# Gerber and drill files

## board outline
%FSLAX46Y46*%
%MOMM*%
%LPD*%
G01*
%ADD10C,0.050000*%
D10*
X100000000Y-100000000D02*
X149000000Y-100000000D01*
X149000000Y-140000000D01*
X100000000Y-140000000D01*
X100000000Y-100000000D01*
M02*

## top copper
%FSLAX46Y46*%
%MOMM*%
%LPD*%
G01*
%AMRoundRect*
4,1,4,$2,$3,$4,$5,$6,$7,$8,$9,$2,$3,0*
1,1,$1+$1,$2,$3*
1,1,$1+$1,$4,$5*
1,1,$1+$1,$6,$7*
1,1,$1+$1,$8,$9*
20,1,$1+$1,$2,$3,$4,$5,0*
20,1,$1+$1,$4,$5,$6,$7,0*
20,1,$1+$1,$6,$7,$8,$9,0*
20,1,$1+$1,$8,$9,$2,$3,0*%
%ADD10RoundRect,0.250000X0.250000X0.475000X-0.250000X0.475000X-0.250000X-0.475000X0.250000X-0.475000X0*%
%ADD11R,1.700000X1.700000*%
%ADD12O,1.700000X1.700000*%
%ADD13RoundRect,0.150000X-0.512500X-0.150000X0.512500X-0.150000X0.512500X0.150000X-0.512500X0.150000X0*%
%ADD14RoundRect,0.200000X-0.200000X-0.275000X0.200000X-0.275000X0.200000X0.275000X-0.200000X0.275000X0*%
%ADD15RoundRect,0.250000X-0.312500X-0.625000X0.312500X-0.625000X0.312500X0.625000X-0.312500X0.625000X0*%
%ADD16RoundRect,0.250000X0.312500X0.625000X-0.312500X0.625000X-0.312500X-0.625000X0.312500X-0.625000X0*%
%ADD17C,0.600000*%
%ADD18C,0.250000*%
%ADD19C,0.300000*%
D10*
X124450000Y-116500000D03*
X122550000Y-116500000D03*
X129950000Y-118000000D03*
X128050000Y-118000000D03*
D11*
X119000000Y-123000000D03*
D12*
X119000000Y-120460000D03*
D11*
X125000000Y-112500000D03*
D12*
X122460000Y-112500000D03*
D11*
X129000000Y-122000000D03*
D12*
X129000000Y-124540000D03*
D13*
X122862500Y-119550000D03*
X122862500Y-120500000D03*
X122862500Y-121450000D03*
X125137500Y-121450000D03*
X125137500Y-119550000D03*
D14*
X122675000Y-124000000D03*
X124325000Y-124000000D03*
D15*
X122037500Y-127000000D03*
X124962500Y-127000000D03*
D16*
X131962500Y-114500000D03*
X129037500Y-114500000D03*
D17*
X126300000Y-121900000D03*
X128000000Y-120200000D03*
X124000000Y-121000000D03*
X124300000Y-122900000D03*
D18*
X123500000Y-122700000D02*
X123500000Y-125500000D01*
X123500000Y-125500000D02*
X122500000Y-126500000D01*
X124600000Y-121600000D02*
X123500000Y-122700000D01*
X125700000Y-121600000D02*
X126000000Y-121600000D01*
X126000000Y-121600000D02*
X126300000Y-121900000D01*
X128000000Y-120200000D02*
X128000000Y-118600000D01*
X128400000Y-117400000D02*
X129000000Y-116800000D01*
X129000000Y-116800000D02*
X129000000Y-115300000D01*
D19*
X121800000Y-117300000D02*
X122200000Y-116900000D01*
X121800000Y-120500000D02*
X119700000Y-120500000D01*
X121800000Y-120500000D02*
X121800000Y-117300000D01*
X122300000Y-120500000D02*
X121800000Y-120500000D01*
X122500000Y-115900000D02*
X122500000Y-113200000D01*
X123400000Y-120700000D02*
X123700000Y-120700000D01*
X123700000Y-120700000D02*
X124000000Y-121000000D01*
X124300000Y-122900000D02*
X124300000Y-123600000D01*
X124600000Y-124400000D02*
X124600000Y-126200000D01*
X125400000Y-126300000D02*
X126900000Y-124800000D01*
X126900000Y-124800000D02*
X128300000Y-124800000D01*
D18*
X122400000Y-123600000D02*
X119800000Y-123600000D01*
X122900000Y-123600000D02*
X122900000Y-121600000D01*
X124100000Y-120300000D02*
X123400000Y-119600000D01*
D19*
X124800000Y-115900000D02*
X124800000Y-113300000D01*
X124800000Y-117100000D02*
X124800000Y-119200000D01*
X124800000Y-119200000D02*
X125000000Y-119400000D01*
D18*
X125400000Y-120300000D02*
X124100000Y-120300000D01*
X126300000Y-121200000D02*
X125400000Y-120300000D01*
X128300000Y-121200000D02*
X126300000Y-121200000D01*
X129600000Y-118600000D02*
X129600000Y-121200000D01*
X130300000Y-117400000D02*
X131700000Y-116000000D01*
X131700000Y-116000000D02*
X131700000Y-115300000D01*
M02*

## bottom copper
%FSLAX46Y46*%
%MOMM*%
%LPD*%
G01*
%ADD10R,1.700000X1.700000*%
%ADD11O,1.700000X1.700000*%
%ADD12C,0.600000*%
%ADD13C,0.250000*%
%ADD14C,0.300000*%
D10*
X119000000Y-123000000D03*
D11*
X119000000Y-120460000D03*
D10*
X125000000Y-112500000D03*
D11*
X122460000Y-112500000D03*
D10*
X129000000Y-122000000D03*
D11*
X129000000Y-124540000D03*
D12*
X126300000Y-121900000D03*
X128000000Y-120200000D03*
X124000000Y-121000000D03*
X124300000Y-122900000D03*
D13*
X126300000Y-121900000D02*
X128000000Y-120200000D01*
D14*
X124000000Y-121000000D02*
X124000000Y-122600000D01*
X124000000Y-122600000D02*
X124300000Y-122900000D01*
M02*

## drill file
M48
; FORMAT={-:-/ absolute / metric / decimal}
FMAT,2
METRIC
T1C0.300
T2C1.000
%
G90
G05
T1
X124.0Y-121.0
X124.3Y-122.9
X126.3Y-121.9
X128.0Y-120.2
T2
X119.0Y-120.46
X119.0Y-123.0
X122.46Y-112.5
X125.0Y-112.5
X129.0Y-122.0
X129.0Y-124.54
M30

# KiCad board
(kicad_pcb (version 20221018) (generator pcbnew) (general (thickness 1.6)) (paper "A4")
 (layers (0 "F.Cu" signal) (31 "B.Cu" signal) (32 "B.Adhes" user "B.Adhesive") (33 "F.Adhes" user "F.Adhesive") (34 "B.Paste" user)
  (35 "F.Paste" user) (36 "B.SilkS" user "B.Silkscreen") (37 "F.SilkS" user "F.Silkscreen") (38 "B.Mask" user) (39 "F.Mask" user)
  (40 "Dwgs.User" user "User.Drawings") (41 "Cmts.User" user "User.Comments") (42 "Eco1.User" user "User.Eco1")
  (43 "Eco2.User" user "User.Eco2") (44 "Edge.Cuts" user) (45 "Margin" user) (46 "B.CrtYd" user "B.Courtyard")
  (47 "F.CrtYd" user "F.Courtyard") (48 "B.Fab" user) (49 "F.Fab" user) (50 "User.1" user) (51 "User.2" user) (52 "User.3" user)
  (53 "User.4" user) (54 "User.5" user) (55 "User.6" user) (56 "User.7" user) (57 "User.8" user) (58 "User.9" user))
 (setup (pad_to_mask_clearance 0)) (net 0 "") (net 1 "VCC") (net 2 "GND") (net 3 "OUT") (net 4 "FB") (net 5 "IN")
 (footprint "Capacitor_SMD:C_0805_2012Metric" (layer "F.Cu") (at 123.5 116.5 180)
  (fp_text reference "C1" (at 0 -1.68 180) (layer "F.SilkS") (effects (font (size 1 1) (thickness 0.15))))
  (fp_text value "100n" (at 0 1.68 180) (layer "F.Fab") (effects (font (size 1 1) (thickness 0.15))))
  (pad "1" smd roundrect (at -0.95 0 180) (size 1 1.45) (layers "F.Cu" "F.Paste" "F.Mask") (roundrect_rratio 0.25) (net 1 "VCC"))
  (pad "2" smd roundrect (at 0.95 0 180) (size 1 1.45) (layers "F.Cu" "F.Paste" "F.Mask") (roundrect_rratio 0.25) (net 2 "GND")))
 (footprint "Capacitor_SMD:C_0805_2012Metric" (layer "F.Cu") (at 129 118 180)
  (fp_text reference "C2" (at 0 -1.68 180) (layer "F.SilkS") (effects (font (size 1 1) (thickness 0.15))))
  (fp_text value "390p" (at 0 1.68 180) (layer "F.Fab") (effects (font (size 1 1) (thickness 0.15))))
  (pad "1" smd roundrect (at -0.95 0 180) (size 1 1.45) (layers "F.Cu" "F.Paste" "F.Mask") (roundrect_rratio 0.25) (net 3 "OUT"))
  (pad "2" smd roundrect (at 0.95 0 180) (size 1 1.45) (layers "F.Cu" "F.Paste" "F.Mask") (roundrect_rratio 0.25) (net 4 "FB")))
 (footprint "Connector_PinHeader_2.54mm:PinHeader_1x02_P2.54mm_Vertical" (layer "F.Cu") (at 119 123 180)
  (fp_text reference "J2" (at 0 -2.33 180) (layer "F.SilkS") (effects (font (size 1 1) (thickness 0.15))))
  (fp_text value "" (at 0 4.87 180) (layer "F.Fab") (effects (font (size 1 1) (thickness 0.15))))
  (pad "1" thru_hole rect (at 0 0 180) (size 1.7 1.7) (drill 1) (layers "*.Cu" "*.Mask") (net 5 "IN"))
  (pad "2" thru_hole oval (at 0 2.54 180) (size 1.7 1.7) (drill 1) (layers "*.Cu" "*.Mask") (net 2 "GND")))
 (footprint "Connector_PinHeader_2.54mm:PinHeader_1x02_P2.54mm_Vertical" (layer "F.Cu") (at 125 112.5 -90)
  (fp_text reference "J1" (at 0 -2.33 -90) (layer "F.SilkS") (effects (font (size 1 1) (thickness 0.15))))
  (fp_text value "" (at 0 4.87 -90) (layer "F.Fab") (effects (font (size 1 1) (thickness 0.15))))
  (pad "1" thru_hole rect (at 0 0 270) (size 1.7 1.7) (drill 1) (layers "*.Cu" "*.Mask") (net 1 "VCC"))
  (pad "2" thru_hole oval (at 0 2.54 270) (size 1.7 1.7) (drill 1) (layers "*.Cu" "*.Mask") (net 2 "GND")))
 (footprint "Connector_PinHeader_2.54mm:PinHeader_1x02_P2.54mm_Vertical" (layer "F.Cu") (at 129 122)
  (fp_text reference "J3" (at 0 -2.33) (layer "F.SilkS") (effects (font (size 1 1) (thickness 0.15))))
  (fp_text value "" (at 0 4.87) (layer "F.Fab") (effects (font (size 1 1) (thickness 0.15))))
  (pad "1" thru_hole rect (at 0 0) (size 1.7 1.7) (drill 1) (layers "*.Cu" "*.Mask") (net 3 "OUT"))
  (pad "2" thru_hole oval (at 0 2.54) (size 1.7 1.7) (drill 1) (layers "*.Cu" "*.Mask") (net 2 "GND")))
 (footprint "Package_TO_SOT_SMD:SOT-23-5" (layer "F.Cu") (at 124 120.5)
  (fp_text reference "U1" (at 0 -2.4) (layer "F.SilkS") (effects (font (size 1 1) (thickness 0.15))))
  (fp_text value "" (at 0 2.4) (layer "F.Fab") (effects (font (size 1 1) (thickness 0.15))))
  (pad "1" smd roundrect (at -1.1375 -0.95) (size 1.325 0.6) (layers "F.Cu" "F.Paste" "F.Mask") (roundrect_rratio 0.25) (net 3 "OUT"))
  (pad "2" smd roundrect (at -1.1375 0) (size 1.325 0.6) (layers "F.Cu" "F.Paste" "F.Mask") (roundrect_rratio 0.25) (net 2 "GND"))
  (pad "3" smd roundrect (at -1.1375 0.95) (size 1.325 0.6) (layers "F.Cu" "F.Paste" "F.Mask") (roundrect_rratio 0.25) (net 5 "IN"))
  (pad "4" smd roundrect (at 1.1375 0.95) (size 1.325 0.6) (layers "F.Cu" "F.Paste" "F.Mask") (roundrect_rratio 0.25) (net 4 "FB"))
  (pad "5" smd roundrect (at 1.1375 -0.95) (size 1.325 0.6) (layers "F.Cu" "F.Paste" "F.Mask") (roundrect_rratio 0.25) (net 1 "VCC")))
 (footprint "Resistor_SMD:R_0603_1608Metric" (layer "F.Cu") (at 123.5 124)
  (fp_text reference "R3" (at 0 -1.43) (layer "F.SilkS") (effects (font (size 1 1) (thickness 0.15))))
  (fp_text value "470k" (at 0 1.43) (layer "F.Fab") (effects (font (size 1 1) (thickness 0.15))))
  (pad "1" smd roundrect (at -0.825 0) (size 0.8 0.95) (layers "F.Cu" "F.Paste" "F.Mask") (roundrect_rratio 0.25) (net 5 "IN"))
  (pad "2" smd roundrect (at 0.825 0) (size 0.8 0.95) (layers "F.Cu" "F.Paste" "F.Mask") (roundrect_rratio 0.25) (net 2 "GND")))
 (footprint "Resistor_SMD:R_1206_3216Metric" (layer "F.Cu") (at 123.5 127)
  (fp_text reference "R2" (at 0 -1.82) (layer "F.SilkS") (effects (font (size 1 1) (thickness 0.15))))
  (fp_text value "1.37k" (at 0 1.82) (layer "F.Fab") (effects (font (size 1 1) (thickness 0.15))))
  (pad "1" smd roundrect (at -1.4625 0) (size 1.125 1.75) (layers "F.Cu" "F.Paste" "F.Mask") (roundrect_rratio 0.222222) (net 4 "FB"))
  (pad "2" smd roundrect (at 1.4625 0) (size 1.125 1.75) (layers "F.Cu" "F.Paste" "F.Mask") (roundrect_rratio 0.222222) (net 2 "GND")))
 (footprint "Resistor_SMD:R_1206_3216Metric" (layer "F.Cu") (at 130.5 114.5 180)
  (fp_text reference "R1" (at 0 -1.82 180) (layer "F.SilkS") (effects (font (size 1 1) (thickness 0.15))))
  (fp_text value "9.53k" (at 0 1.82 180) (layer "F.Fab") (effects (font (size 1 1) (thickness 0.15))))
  (pad "1" smd roundrect (at -1.4625 0 180) (size 1.125 1.75) (layers "F.Cu" "F.Paste" "F.Mask") (roundrect_rratio 0.222222) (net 3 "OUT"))
  (pad "2" smd roundrect (at 1.4625 0 180) (size 1.125 1.75) (layers "F.Cu" "F.Paste" "F.Mask") (roundrect_rratio 0.222222) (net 4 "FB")))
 (gr_rect (start 100 100) (end 149 140) (stroke (width 0.05) (type default)) (fill none) (layer "Edge.Cuts"))
 (segment (start 123.5 122.7) (end 123.5 125.5) (width 0.25) (layer "F.Cu") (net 4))
 (segment (start 123.5 125.5) (end 122.5 126.5) (width 0.25) (layer "F.Cu") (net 4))
 (segment (start 124.6 121.6) (end 123.5 122.7) (width 0.25) (layer "F.Cu") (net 4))
 (segment (start 125.7 121.6) (end 126 121.6) (width 0.25) (layer "F.Cu") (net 4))
 (segment (start 126 121.6) (end 126.3 121.9) (width 0.25) (layer "F.Cu") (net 4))
 (segment (start 128 120.2) (end 128 118.6) (width 0.25) (layer "F.Cu") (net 4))
 (segment (start 128.4 117.4) (end 129 116.8) (width 0.25) (layer "F.Cu") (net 4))
 (segment (start 129 116.8) (end 129 115.3) (width 0.25) (layer "F.Cu") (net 4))
 (via (at 126.3 121.9) (size 0.6) (drill 0.3) (layers "F.Cu" "B.Cu") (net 4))
 (via (at 128 120.2) (size 0.6) (drill 0.3) (layers "F.Cu" "B.Cu") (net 4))
 (segment (start 121.8 117.3) (end 122.2 116.9) (width 0.3) (layer "F.Cu") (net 2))
 (segment (start 121.8 120.5) (end 119.7 120.5) (width 0.3) (layer "F.Cu") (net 2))
 (segment (start 121.8 120.5) (end 121.8 117.3) (width 0.3) (layer "F.Cu") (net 2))
 (segment (start 122.3 120.5) (end 121.8 120.5) (width 0.3) (layer "F.Cu") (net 2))
 (segment (start 122.5 115.9) (end 122.5 113.2) (width 0.3) (layer "F.Cu") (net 2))
 (segment (start 123.4 120.7) (end 123.7 120.7) (width 0.3) (layer "F.Cu") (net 2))
 (segment (start 123.7 120.7) (end 124 121) (width 0.3) (layer "F.Cu") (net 2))
 (segment (start 124.3 122.9) (end 124.3 123.6) (width 0.3) (layer "F.Cu") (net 2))
 (segment (start 124.6 124.4) (end 124.6 126.2) (width 0.3) (layer "F.Cu") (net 2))
 (segment (start 125.4 126.3) (end 126.9 124.8) (width 0.3) (layer "F.Cu") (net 2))
 (segment (start 126.3 121.9) (end 128 120.2) (width 0.25) (layer "B.Cu") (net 4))
 (segment (start 126.9 124.8) (end 128.3 124.8) (width 0.3) (layer "F.Cu") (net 2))
 (via (at 124 121) (size 0.6) (drill 0.3) (layers "F.Cu" "B.Cu") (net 2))
 (via (at 124.3 122.9) (size 0.6) (drill 0.3) (layers "F.Cu" "B.Cu") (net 2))
 (segment (start 122.4 123.6) (end 119.8 123.6) (width 0.25) (layer "F.Cu") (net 5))
 (segment (start 122.9 123.6) (end 122.9 121.6) (width 0.25) (layer "F.Cu") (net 5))
 (segment (start 124 121) (end 124 122.6) (width 0.3) (layer "B.Cu") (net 2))
 (segment (start 124 122.6) (end 124.3 122.9) (width 0.3) (layer "B.Cu") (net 2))
 (segment (start 124.1 120.3) (end 123.4 119.6) (width 0.25) (layer "F.Cu") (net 3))
 (segment (start 124.8 115.9) (end 124.8 113.3) (width 0.3) (layer "F.Cu") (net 1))
 (segment (start 124.8 117.1) (end 124.8 119.2) (width 0.3) (layer "F.Cu") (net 1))
 (segment (start 124.8 119.2) (end 125 119.4) (width 0.3) (layer "F.Cu") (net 1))
 (segment (start 125.4 120.3) (end 124.1 120.3) (width 0.25) (layer "F.Cu") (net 3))
 (segment (start 126.3 121.2) (end 125.4 120.3) (width 0.25) (layer "F.Cu") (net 3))
 (segment (start 128.3 121.2) (end 126.3 121.2) (width 0.25) (layer "F.Cu") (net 3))
 (segment (start 129.6 118.6) (end 129.6 121.2) (width 0.25) (layer "F.Cu") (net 3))
 (segment (start 130.3 117.4) (end 131.7 116) (width 0.25) (layer "F.Cu") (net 3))
 (segment (start 131.7 116) (end 131.7 115.3) (width 0.25) (layer "F.Cu") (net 3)))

